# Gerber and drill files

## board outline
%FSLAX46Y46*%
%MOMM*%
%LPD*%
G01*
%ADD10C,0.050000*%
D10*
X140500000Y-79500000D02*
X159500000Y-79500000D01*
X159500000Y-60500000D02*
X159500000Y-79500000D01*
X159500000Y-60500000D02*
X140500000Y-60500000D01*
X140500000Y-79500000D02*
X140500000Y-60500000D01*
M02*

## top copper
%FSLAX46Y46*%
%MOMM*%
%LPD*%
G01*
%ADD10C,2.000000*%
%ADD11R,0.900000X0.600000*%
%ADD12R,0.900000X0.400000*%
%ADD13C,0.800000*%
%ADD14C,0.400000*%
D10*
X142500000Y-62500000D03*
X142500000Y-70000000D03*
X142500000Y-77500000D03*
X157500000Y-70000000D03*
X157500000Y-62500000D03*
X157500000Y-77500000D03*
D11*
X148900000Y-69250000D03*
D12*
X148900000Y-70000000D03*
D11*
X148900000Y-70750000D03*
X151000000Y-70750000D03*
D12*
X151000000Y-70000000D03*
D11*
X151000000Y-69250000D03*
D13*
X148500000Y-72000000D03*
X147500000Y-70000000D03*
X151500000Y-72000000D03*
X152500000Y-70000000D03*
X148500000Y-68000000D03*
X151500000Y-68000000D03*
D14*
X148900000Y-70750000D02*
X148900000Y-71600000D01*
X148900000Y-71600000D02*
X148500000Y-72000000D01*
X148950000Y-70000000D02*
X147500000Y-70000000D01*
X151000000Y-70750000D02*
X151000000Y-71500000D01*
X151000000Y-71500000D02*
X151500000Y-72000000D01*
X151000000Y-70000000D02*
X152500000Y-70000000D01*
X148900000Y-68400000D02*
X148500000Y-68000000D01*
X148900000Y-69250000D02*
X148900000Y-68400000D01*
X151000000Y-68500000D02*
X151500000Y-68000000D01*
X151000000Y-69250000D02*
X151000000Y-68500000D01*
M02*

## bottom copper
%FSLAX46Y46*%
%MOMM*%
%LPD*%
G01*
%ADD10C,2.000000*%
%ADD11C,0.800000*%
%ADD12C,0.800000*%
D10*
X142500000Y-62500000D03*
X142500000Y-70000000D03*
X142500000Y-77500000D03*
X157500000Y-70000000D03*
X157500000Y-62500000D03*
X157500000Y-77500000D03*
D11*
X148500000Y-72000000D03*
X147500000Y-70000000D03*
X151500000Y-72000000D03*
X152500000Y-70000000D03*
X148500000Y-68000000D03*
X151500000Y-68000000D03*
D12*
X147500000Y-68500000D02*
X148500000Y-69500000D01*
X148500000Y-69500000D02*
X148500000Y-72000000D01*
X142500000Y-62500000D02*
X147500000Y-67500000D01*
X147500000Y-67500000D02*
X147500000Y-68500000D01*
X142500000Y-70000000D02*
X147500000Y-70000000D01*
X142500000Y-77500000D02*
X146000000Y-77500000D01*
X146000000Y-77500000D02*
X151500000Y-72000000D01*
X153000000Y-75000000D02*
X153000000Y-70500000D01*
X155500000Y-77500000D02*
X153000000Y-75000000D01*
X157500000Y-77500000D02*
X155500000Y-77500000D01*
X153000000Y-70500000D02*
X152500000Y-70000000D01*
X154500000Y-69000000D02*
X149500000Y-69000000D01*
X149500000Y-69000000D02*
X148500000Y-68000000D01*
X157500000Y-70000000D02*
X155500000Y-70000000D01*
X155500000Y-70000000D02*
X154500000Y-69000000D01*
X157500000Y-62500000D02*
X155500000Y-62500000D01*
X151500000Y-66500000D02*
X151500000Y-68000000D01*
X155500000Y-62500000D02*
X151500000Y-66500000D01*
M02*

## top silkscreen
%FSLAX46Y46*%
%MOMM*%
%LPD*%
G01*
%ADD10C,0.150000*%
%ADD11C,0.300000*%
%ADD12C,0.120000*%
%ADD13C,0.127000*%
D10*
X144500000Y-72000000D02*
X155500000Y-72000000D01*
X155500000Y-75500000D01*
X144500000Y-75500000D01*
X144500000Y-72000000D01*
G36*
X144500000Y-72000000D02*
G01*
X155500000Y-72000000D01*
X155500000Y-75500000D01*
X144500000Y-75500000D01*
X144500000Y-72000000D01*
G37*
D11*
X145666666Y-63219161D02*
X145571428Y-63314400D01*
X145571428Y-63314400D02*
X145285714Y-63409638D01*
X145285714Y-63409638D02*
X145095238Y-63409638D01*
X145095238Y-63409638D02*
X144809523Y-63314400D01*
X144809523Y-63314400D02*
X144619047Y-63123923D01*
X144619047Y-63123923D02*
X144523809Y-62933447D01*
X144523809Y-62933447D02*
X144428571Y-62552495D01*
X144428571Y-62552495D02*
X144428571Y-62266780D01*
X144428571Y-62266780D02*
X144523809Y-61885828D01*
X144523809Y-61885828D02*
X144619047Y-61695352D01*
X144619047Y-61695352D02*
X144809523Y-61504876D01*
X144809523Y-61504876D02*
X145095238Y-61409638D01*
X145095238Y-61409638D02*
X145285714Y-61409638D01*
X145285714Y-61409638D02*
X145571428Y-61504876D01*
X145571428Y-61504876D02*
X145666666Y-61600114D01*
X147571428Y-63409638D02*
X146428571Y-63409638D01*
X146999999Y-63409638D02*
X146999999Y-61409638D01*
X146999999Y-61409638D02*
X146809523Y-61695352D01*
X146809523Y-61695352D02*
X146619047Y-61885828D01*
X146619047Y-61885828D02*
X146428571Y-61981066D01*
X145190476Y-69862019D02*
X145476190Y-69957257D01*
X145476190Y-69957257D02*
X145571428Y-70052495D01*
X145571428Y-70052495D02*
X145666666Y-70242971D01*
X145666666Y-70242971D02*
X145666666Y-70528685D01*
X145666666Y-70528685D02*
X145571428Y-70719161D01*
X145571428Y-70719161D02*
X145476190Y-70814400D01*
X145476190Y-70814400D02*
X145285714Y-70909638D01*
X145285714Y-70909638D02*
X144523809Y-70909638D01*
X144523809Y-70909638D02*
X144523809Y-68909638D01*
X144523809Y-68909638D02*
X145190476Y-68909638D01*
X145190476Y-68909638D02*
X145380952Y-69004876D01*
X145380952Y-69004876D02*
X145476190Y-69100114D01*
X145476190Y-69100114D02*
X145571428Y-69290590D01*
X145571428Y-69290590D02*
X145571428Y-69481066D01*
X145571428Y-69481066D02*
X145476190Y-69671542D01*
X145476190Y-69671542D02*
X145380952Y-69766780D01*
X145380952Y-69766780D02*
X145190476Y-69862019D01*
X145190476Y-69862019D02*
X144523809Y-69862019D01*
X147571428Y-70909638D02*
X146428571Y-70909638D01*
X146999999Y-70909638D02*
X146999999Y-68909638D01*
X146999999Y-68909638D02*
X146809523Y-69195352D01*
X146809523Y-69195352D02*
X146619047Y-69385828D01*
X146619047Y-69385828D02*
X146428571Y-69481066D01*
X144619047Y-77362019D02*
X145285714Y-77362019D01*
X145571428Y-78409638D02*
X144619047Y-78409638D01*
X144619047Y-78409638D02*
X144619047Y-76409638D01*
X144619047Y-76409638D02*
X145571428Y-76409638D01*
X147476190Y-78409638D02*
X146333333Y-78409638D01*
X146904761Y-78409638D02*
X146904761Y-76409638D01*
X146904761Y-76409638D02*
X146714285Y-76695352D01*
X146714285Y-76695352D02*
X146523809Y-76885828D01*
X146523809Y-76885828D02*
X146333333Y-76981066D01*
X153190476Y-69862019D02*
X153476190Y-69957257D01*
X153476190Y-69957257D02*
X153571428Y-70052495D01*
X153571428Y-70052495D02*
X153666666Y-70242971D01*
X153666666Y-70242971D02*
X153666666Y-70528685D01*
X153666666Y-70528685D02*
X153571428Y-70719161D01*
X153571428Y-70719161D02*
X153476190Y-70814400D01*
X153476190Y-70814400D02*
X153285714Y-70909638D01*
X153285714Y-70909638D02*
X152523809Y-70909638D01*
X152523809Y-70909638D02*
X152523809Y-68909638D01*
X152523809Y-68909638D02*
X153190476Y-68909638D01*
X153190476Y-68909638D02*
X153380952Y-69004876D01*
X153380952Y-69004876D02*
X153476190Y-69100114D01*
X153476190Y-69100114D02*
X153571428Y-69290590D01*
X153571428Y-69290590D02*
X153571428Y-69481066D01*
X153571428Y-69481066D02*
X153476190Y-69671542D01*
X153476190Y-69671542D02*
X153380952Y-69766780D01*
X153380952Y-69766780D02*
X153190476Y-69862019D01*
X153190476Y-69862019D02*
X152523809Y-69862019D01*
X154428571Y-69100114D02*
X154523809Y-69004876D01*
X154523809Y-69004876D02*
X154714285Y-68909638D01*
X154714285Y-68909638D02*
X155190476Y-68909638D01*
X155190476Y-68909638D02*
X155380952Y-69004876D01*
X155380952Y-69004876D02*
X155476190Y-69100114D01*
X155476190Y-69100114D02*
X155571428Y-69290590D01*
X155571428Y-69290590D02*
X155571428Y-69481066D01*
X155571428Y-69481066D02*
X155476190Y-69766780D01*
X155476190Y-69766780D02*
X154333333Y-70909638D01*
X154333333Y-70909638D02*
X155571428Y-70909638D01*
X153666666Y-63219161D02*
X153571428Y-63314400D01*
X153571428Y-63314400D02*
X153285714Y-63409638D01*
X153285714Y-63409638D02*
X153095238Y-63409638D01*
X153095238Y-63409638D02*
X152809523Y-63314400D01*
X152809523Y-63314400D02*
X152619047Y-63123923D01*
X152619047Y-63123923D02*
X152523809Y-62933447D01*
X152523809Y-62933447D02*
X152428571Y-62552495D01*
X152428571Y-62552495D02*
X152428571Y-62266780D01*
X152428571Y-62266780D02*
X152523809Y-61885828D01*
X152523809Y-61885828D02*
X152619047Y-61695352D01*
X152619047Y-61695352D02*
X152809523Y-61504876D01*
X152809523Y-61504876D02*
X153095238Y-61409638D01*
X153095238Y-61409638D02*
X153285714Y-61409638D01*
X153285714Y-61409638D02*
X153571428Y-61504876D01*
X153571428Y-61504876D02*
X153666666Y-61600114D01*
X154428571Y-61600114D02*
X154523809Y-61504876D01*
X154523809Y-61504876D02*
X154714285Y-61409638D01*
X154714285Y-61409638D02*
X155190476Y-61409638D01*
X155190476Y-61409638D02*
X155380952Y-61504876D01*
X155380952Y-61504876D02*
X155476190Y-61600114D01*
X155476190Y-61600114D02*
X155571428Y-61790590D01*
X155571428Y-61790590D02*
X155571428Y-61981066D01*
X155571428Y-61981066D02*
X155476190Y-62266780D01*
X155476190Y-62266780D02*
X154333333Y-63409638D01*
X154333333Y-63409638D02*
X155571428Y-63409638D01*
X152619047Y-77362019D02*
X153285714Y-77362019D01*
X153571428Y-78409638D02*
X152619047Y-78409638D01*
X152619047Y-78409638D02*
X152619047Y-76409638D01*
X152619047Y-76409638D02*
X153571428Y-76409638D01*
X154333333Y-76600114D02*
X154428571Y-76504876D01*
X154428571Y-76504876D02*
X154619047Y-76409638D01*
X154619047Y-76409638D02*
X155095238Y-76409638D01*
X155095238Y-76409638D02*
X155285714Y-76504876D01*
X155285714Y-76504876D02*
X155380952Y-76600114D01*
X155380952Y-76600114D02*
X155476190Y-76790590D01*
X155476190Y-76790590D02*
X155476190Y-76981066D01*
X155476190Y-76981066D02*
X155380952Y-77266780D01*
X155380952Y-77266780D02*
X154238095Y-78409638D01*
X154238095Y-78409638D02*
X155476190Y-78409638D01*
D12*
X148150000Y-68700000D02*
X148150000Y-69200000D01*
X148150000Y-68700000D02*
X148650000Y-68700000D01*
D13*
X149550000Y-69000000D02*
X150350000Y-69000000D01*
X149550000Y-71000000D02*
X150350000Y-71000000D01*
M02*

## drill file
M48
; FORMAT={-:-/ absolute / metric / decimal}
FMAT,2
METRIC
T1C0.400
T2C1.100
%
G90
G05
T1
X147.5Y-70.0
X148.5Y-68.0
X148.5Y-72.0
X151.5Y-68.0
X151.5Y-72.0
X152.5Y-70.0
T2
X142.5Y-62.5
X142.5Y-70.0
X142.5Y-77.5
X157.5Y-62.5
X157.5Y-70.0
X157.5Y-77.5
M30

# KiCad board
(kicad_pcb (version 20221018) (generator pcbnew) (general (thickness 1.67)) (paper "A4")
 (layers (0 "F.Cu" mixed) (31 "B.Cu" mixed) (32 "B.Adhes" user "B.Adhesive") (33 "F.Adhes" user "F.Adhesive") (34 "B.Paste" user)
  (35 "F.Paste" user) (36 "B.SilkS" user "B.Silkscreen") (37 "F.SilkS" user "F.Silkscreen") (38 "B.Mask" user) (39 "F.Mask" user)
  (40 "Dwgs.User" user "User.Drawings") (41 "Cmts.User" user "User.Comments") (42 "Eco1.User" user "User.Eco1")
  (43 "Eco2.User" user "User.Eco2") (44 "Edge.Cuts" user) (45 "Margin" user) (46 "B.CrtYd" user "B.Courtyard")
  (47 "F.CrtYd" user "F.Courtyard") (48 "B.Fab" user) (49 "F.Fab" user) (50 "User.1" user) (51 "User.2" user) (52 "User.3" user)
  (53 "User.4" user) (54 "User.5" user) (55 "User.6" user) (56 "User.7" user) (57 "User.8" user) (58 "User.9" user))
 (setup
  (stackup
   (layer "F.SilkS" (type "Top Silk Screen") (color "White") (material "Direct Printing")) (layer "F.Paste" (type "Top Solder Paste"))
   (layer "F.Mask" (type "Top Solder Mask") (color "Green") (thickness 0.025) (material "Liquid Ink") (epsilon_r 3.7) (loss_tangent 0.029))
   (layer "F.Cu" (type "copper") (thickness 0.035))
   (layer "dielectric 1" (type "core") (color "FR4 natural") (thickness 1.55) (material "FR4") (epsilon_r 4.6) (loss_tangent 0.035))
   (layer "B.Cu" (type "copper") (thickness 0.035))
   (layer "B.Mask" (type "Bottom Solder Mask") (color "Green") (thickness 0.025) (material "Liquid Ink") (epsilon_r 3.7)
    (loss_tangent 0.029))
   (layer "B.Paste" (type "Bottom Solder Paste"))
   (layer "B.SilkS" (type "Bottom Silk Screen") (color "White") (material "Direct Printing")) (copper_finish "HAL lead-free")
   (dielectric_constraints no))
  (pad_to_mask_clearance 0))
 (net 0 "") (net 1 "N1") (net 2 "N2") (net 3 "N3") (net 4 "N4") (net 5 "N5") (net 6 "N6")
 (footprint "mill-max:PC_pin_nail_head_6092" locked (layer "F.Cu") (at 142.5 62.5)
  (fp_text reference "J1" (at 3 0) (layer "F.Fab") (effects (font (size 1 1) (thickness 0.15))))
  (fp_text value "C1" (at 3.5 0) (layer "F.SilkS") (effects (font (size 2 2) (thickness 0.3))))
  (pad "1" thru_hole circle locked (at 0 0) (size 2 2) (drill 1.1) (layers "*.Cu" "*.Mask") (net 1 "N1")))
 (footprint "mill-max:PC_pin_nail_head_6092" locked (layer "F.Cu") (at 142.5 70)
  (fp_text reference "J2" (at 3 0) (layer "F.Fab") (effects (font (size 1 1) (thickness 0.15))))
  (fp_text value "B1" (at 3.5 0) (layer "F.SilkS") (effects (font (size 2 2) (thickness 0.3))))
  (pad "1" thru_hole circle locked (at 0 0) (size 2 2) (drill 1.1) (layers "*.Cu" "*.Mask") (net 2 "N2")))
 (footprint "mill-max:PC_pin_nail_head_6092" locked (layer "F.Cu") (at 142.5 77.5)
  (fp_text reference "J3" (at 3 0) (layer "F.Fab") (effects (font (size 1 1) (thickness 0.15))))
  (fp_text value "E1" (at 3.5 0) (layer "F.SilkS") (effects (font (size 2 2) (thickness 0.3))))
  (pad "1" thru_hole circle locked (at 0 0) (size 2 2) (drill 1.1) (layers "*.Cu" "*.Mask") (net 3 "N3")))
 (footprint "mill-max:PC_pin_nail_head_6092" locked (layer "F.Cu") (at 157.5 70)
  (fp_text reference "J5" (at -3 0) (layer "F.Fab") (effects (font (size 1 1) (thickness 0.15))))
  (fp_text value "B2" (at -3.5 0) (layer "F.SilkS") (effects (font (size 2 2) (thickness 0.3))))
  (pad "1" thru_hole circle locked (at 0 0) (size 2 2) (drill 1.1) (layers "*.Cu" "*.Mask") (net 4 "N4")))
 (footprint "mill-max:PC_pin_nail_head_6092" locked (layer "F.Cu") (at 157.5 62.5)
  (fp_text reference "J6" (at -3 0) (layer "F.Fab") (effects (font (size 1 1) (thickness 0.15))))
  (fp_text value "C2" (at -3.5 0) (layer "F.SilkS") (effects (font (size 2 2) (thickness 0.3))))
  (pad "1" thru_hole circle locked (at 0 0) (size 2 2) (drill 1.1) (layers "*.Cu" "*.Mask") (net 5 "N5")))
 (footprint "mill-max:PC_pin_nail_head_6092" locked (layer "F.Cu") (at 157.5 77.5)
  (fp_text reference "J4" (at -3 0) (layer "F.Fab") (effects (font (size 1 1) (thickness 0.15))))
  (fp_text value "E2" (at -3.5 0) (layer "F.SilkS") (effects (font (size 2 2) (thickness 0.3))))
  (pad "1" thru_hole circle locked (at 0 0) (size 2 2) (drill 1.1) (layers "*.Cu" "*.Mask") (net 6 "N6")))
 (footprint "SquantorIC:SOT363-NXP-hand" (layer "F.Cu") (at 149.95 70)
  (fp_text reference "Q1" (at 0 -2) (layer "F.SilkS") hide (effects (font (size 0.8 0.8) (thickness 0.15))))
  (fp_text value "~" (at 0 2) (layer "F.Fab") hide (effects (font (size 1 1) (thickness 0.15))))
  (fp_line (start -1.8 -1.3) (end -1.8 -0.8) (stroke (width 0.12) (type solid)) (layer "F.SilkS"))
  (fp_line (start -1.8 -1.3) (end -1.3 -1.3) (stroke (width 0.12) (type solid)) (layer "F.SilkS"))
  (fp_line (start -0.4 -1) (end 0.4 -1) (stroke (width 0.127) (type solid)) (layer "F.SilkS"))
  (fp_line (start -0.4 1) (end 0.4 1) (stroke (width 0.127) (type solid)) (layer "F.SilkS"))
  (pad "1" smd rect (at -1.05 -0.75 270) (size 0.6 0.9) (layers "F.Cu" "F.Paste" "F.Mask") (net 4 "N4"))
  (pad "2" smd rect (at -1.05 0 270) (size 0.4 0.9) (layers "F.Cu" "F.Paste" "F.Mask") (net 2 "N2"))
  (pad "3" smd rect (at -1.05 0.75 270) (size 0.6 0.9) (layers "F.Cu" "F.Paste" "F.Mask") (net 1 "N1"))
  (pad "4" smd rect (at 1.05 0.75 270) (size 0.6 0.9) (layers "F.Cu" "F.Paste" "F.Mask") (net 3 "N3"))
  (pad "5" smd rect (at 1.05 0 270) (size 0.4 0.9) (layers "F.Cu" "F.Paste" "F.Mask") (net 6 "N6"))
  (pad "6" smd rect (at 1.05 -0.75 270) (size 0.6 0.9) (layers "F.Cu" "F.Paste" "F.Mask") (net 5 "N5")))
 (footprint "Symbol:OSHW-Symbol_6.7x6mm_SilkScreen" (layer "B.Cu") (at 150 74.8 180)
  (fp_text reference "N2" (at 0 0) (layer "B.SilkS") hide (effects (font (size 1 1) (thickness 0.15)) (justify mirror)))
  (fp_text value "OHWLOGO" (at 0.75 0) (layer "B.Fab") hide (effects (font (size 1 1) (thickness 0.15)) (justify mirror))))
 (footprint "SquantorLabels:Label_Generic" (layer "B.Cu") (at 150.9 78.5 180)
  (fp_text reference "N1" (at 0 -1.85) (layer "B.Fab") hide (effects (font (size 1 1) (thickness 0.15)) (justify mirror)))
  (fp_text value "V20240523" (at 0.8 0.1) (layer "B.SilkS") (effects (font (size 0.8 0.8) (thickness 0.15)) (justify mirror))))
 (gr_rect (start 144.5 72) (end 155.5 75.5) (stroke (width 0.15) (type solid)) (fill solid) (layer "F.SilkS"))
 (gr_line (start 140.5 79.5) (end 159.5 79.5) (stroke (width 0.05) (type solid)) (layer "Edge.Cuts"))
 (gr_line (start 159.5 60.5) (end 159.5 79.5) (stroke (width 0.05) (type solid)) (layer "Edge.Cuts"))
 (gr_line (start 159.5 60.5) (end 140.5 60.5) (stroke (width 0.05) (type solid)) (layer "Edge.Cuts"))
 (gr_line (start 140.5 79.5) (end 140.5 60.5) (stroke (width 0.05) (type solid)) (layer "Edge.Cuts"))
 (segment (start 148.9 70.75) (end 148.9 71.6) (width 0.4) (layer "F.Cu") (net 1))
 (segment (start 148.9 71.6) (end 148.5 72) (width 0.4) (layer "F.Cu") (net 1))
 (via (at 148.5 72) (size 0.8) (drill 0.4) (layers "F.Cu" "B.Cu") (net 1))
 (segment (start 147.5 68.5) (end 148.5 69.5) (width 0.8) (layer "B.Cu") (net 1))
 (segment (start 148.5 69.5) (end 148.5 72) (width 0.8) (layer "B.Cu") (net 1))
 (segment (start 142.5 62.5) (end 147.5 67.5) (width 0.8) (layer "B.Cu") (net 1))
 (segment (start 147.5 67.5) (end 147.5 68.5) (width 0.8) (layer "B.Cu") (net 1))
 (segment (start 148.95 70) (end 147.5 70) (width 0.4) (layer "F.Cu") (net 2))
 (via (at 147.5 70) (size 0.8) (drill 0.4) (layers "F.Cu" "B.Cu") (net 2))
 (segment (start 142.5 70) (end 147.5 70) (width 0.8) (layer "B.Cu") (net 2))
 (segment (start 151 70.75) (end 151 71.5) (width 0.4) (layer "F.Cu") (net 3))
 (segment (start 151 71.5) (end 151.5 72) (width 0.4) (layer "F.Cu") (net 3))
 (via (at 151.5 72) (size 0.8) (drill 0.4) (layers "F.Cu" "B.Cu") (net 3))
 (segment (start 142.5 77.5) (end 146 77.5) (width 0.8) (layer "B.Cu") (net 3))
 (segment (start 146 77.5) (end 151.5 72) (width 0.8) (layer "B.Cu") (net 3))
 (segment (start 151 70) (end 152.5 70) (width 0.4) (layer "F.Cu") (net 6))
 (via (at 152.5 70) (size 0.8) (drill 0.4) (layers "F.Cu" "B.Cu") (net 6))
 (segment (start 153 75) (end 153 70.5) (width 0.8) (layer "B.Cu") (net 6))
 (segment (start 155.5 77.5) (end 153 75) (width 0.8) (layer "B.Cu") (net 6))
 (segment (start 157.5 77.5) (end 155.5 77.5) (width 0.8) (layer "B.Cu") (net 6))
 (segment (start 153 70.5) (end 152.5 70) (width 0.8) (layer "B.Cu") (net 6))
 (segment (start 148.9 68.4) (end 148.5 68) (width 0.4) (layer "F.Cu") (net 4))
 (segment (start 148.9 69.25) (end 148.9 68.4) (width 0.4) (layer "F.Cu") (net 4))
 (via (at 148.5 68) (size 0.8) (drill 0.4) (layers "F.Cu" "B.Cu") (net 4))
 (segment (start 154.5 69) (end 149.5 69) (width 0.8) (layer "B.Cu") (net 4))
 (segment (start 149.5 69) (end 148.5 68) (width 0.8) (layer "B.Cu") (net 4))
 (segment (start 157.5 70) (end 155.5 70) (width 0.8) (layer "B.Cu") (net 4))
 (segment (start 155.5 70) (end 154.5 69) (width 0.8) (layer "B.Cu") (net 4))
 (segment (start 151 68.5) (end 151.5 68) (width 0.4) (layer "F.Cu") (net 5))
 (segment (start 151 69.25) (end 151 68.5) (width 0.4) (layer "F.Cu") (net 5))
 (via (at 151.5 68) (size 0.8) (drill 0.4) (layers "F.Cu" "B.Cu") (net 5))
 (segment (start 157.5 62.5) (end 155.5 62.5) (width 0.8) (layer "B.Cu") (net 5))
 (segment (start 151.5 66.5) (end 151.5 68) (width 0.8) (layer "B.Cu") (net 5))
 (segment (start 155.5 62.5) (end 151.5 66.5) (width 0.8) (layer "B.Cu") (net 5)))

